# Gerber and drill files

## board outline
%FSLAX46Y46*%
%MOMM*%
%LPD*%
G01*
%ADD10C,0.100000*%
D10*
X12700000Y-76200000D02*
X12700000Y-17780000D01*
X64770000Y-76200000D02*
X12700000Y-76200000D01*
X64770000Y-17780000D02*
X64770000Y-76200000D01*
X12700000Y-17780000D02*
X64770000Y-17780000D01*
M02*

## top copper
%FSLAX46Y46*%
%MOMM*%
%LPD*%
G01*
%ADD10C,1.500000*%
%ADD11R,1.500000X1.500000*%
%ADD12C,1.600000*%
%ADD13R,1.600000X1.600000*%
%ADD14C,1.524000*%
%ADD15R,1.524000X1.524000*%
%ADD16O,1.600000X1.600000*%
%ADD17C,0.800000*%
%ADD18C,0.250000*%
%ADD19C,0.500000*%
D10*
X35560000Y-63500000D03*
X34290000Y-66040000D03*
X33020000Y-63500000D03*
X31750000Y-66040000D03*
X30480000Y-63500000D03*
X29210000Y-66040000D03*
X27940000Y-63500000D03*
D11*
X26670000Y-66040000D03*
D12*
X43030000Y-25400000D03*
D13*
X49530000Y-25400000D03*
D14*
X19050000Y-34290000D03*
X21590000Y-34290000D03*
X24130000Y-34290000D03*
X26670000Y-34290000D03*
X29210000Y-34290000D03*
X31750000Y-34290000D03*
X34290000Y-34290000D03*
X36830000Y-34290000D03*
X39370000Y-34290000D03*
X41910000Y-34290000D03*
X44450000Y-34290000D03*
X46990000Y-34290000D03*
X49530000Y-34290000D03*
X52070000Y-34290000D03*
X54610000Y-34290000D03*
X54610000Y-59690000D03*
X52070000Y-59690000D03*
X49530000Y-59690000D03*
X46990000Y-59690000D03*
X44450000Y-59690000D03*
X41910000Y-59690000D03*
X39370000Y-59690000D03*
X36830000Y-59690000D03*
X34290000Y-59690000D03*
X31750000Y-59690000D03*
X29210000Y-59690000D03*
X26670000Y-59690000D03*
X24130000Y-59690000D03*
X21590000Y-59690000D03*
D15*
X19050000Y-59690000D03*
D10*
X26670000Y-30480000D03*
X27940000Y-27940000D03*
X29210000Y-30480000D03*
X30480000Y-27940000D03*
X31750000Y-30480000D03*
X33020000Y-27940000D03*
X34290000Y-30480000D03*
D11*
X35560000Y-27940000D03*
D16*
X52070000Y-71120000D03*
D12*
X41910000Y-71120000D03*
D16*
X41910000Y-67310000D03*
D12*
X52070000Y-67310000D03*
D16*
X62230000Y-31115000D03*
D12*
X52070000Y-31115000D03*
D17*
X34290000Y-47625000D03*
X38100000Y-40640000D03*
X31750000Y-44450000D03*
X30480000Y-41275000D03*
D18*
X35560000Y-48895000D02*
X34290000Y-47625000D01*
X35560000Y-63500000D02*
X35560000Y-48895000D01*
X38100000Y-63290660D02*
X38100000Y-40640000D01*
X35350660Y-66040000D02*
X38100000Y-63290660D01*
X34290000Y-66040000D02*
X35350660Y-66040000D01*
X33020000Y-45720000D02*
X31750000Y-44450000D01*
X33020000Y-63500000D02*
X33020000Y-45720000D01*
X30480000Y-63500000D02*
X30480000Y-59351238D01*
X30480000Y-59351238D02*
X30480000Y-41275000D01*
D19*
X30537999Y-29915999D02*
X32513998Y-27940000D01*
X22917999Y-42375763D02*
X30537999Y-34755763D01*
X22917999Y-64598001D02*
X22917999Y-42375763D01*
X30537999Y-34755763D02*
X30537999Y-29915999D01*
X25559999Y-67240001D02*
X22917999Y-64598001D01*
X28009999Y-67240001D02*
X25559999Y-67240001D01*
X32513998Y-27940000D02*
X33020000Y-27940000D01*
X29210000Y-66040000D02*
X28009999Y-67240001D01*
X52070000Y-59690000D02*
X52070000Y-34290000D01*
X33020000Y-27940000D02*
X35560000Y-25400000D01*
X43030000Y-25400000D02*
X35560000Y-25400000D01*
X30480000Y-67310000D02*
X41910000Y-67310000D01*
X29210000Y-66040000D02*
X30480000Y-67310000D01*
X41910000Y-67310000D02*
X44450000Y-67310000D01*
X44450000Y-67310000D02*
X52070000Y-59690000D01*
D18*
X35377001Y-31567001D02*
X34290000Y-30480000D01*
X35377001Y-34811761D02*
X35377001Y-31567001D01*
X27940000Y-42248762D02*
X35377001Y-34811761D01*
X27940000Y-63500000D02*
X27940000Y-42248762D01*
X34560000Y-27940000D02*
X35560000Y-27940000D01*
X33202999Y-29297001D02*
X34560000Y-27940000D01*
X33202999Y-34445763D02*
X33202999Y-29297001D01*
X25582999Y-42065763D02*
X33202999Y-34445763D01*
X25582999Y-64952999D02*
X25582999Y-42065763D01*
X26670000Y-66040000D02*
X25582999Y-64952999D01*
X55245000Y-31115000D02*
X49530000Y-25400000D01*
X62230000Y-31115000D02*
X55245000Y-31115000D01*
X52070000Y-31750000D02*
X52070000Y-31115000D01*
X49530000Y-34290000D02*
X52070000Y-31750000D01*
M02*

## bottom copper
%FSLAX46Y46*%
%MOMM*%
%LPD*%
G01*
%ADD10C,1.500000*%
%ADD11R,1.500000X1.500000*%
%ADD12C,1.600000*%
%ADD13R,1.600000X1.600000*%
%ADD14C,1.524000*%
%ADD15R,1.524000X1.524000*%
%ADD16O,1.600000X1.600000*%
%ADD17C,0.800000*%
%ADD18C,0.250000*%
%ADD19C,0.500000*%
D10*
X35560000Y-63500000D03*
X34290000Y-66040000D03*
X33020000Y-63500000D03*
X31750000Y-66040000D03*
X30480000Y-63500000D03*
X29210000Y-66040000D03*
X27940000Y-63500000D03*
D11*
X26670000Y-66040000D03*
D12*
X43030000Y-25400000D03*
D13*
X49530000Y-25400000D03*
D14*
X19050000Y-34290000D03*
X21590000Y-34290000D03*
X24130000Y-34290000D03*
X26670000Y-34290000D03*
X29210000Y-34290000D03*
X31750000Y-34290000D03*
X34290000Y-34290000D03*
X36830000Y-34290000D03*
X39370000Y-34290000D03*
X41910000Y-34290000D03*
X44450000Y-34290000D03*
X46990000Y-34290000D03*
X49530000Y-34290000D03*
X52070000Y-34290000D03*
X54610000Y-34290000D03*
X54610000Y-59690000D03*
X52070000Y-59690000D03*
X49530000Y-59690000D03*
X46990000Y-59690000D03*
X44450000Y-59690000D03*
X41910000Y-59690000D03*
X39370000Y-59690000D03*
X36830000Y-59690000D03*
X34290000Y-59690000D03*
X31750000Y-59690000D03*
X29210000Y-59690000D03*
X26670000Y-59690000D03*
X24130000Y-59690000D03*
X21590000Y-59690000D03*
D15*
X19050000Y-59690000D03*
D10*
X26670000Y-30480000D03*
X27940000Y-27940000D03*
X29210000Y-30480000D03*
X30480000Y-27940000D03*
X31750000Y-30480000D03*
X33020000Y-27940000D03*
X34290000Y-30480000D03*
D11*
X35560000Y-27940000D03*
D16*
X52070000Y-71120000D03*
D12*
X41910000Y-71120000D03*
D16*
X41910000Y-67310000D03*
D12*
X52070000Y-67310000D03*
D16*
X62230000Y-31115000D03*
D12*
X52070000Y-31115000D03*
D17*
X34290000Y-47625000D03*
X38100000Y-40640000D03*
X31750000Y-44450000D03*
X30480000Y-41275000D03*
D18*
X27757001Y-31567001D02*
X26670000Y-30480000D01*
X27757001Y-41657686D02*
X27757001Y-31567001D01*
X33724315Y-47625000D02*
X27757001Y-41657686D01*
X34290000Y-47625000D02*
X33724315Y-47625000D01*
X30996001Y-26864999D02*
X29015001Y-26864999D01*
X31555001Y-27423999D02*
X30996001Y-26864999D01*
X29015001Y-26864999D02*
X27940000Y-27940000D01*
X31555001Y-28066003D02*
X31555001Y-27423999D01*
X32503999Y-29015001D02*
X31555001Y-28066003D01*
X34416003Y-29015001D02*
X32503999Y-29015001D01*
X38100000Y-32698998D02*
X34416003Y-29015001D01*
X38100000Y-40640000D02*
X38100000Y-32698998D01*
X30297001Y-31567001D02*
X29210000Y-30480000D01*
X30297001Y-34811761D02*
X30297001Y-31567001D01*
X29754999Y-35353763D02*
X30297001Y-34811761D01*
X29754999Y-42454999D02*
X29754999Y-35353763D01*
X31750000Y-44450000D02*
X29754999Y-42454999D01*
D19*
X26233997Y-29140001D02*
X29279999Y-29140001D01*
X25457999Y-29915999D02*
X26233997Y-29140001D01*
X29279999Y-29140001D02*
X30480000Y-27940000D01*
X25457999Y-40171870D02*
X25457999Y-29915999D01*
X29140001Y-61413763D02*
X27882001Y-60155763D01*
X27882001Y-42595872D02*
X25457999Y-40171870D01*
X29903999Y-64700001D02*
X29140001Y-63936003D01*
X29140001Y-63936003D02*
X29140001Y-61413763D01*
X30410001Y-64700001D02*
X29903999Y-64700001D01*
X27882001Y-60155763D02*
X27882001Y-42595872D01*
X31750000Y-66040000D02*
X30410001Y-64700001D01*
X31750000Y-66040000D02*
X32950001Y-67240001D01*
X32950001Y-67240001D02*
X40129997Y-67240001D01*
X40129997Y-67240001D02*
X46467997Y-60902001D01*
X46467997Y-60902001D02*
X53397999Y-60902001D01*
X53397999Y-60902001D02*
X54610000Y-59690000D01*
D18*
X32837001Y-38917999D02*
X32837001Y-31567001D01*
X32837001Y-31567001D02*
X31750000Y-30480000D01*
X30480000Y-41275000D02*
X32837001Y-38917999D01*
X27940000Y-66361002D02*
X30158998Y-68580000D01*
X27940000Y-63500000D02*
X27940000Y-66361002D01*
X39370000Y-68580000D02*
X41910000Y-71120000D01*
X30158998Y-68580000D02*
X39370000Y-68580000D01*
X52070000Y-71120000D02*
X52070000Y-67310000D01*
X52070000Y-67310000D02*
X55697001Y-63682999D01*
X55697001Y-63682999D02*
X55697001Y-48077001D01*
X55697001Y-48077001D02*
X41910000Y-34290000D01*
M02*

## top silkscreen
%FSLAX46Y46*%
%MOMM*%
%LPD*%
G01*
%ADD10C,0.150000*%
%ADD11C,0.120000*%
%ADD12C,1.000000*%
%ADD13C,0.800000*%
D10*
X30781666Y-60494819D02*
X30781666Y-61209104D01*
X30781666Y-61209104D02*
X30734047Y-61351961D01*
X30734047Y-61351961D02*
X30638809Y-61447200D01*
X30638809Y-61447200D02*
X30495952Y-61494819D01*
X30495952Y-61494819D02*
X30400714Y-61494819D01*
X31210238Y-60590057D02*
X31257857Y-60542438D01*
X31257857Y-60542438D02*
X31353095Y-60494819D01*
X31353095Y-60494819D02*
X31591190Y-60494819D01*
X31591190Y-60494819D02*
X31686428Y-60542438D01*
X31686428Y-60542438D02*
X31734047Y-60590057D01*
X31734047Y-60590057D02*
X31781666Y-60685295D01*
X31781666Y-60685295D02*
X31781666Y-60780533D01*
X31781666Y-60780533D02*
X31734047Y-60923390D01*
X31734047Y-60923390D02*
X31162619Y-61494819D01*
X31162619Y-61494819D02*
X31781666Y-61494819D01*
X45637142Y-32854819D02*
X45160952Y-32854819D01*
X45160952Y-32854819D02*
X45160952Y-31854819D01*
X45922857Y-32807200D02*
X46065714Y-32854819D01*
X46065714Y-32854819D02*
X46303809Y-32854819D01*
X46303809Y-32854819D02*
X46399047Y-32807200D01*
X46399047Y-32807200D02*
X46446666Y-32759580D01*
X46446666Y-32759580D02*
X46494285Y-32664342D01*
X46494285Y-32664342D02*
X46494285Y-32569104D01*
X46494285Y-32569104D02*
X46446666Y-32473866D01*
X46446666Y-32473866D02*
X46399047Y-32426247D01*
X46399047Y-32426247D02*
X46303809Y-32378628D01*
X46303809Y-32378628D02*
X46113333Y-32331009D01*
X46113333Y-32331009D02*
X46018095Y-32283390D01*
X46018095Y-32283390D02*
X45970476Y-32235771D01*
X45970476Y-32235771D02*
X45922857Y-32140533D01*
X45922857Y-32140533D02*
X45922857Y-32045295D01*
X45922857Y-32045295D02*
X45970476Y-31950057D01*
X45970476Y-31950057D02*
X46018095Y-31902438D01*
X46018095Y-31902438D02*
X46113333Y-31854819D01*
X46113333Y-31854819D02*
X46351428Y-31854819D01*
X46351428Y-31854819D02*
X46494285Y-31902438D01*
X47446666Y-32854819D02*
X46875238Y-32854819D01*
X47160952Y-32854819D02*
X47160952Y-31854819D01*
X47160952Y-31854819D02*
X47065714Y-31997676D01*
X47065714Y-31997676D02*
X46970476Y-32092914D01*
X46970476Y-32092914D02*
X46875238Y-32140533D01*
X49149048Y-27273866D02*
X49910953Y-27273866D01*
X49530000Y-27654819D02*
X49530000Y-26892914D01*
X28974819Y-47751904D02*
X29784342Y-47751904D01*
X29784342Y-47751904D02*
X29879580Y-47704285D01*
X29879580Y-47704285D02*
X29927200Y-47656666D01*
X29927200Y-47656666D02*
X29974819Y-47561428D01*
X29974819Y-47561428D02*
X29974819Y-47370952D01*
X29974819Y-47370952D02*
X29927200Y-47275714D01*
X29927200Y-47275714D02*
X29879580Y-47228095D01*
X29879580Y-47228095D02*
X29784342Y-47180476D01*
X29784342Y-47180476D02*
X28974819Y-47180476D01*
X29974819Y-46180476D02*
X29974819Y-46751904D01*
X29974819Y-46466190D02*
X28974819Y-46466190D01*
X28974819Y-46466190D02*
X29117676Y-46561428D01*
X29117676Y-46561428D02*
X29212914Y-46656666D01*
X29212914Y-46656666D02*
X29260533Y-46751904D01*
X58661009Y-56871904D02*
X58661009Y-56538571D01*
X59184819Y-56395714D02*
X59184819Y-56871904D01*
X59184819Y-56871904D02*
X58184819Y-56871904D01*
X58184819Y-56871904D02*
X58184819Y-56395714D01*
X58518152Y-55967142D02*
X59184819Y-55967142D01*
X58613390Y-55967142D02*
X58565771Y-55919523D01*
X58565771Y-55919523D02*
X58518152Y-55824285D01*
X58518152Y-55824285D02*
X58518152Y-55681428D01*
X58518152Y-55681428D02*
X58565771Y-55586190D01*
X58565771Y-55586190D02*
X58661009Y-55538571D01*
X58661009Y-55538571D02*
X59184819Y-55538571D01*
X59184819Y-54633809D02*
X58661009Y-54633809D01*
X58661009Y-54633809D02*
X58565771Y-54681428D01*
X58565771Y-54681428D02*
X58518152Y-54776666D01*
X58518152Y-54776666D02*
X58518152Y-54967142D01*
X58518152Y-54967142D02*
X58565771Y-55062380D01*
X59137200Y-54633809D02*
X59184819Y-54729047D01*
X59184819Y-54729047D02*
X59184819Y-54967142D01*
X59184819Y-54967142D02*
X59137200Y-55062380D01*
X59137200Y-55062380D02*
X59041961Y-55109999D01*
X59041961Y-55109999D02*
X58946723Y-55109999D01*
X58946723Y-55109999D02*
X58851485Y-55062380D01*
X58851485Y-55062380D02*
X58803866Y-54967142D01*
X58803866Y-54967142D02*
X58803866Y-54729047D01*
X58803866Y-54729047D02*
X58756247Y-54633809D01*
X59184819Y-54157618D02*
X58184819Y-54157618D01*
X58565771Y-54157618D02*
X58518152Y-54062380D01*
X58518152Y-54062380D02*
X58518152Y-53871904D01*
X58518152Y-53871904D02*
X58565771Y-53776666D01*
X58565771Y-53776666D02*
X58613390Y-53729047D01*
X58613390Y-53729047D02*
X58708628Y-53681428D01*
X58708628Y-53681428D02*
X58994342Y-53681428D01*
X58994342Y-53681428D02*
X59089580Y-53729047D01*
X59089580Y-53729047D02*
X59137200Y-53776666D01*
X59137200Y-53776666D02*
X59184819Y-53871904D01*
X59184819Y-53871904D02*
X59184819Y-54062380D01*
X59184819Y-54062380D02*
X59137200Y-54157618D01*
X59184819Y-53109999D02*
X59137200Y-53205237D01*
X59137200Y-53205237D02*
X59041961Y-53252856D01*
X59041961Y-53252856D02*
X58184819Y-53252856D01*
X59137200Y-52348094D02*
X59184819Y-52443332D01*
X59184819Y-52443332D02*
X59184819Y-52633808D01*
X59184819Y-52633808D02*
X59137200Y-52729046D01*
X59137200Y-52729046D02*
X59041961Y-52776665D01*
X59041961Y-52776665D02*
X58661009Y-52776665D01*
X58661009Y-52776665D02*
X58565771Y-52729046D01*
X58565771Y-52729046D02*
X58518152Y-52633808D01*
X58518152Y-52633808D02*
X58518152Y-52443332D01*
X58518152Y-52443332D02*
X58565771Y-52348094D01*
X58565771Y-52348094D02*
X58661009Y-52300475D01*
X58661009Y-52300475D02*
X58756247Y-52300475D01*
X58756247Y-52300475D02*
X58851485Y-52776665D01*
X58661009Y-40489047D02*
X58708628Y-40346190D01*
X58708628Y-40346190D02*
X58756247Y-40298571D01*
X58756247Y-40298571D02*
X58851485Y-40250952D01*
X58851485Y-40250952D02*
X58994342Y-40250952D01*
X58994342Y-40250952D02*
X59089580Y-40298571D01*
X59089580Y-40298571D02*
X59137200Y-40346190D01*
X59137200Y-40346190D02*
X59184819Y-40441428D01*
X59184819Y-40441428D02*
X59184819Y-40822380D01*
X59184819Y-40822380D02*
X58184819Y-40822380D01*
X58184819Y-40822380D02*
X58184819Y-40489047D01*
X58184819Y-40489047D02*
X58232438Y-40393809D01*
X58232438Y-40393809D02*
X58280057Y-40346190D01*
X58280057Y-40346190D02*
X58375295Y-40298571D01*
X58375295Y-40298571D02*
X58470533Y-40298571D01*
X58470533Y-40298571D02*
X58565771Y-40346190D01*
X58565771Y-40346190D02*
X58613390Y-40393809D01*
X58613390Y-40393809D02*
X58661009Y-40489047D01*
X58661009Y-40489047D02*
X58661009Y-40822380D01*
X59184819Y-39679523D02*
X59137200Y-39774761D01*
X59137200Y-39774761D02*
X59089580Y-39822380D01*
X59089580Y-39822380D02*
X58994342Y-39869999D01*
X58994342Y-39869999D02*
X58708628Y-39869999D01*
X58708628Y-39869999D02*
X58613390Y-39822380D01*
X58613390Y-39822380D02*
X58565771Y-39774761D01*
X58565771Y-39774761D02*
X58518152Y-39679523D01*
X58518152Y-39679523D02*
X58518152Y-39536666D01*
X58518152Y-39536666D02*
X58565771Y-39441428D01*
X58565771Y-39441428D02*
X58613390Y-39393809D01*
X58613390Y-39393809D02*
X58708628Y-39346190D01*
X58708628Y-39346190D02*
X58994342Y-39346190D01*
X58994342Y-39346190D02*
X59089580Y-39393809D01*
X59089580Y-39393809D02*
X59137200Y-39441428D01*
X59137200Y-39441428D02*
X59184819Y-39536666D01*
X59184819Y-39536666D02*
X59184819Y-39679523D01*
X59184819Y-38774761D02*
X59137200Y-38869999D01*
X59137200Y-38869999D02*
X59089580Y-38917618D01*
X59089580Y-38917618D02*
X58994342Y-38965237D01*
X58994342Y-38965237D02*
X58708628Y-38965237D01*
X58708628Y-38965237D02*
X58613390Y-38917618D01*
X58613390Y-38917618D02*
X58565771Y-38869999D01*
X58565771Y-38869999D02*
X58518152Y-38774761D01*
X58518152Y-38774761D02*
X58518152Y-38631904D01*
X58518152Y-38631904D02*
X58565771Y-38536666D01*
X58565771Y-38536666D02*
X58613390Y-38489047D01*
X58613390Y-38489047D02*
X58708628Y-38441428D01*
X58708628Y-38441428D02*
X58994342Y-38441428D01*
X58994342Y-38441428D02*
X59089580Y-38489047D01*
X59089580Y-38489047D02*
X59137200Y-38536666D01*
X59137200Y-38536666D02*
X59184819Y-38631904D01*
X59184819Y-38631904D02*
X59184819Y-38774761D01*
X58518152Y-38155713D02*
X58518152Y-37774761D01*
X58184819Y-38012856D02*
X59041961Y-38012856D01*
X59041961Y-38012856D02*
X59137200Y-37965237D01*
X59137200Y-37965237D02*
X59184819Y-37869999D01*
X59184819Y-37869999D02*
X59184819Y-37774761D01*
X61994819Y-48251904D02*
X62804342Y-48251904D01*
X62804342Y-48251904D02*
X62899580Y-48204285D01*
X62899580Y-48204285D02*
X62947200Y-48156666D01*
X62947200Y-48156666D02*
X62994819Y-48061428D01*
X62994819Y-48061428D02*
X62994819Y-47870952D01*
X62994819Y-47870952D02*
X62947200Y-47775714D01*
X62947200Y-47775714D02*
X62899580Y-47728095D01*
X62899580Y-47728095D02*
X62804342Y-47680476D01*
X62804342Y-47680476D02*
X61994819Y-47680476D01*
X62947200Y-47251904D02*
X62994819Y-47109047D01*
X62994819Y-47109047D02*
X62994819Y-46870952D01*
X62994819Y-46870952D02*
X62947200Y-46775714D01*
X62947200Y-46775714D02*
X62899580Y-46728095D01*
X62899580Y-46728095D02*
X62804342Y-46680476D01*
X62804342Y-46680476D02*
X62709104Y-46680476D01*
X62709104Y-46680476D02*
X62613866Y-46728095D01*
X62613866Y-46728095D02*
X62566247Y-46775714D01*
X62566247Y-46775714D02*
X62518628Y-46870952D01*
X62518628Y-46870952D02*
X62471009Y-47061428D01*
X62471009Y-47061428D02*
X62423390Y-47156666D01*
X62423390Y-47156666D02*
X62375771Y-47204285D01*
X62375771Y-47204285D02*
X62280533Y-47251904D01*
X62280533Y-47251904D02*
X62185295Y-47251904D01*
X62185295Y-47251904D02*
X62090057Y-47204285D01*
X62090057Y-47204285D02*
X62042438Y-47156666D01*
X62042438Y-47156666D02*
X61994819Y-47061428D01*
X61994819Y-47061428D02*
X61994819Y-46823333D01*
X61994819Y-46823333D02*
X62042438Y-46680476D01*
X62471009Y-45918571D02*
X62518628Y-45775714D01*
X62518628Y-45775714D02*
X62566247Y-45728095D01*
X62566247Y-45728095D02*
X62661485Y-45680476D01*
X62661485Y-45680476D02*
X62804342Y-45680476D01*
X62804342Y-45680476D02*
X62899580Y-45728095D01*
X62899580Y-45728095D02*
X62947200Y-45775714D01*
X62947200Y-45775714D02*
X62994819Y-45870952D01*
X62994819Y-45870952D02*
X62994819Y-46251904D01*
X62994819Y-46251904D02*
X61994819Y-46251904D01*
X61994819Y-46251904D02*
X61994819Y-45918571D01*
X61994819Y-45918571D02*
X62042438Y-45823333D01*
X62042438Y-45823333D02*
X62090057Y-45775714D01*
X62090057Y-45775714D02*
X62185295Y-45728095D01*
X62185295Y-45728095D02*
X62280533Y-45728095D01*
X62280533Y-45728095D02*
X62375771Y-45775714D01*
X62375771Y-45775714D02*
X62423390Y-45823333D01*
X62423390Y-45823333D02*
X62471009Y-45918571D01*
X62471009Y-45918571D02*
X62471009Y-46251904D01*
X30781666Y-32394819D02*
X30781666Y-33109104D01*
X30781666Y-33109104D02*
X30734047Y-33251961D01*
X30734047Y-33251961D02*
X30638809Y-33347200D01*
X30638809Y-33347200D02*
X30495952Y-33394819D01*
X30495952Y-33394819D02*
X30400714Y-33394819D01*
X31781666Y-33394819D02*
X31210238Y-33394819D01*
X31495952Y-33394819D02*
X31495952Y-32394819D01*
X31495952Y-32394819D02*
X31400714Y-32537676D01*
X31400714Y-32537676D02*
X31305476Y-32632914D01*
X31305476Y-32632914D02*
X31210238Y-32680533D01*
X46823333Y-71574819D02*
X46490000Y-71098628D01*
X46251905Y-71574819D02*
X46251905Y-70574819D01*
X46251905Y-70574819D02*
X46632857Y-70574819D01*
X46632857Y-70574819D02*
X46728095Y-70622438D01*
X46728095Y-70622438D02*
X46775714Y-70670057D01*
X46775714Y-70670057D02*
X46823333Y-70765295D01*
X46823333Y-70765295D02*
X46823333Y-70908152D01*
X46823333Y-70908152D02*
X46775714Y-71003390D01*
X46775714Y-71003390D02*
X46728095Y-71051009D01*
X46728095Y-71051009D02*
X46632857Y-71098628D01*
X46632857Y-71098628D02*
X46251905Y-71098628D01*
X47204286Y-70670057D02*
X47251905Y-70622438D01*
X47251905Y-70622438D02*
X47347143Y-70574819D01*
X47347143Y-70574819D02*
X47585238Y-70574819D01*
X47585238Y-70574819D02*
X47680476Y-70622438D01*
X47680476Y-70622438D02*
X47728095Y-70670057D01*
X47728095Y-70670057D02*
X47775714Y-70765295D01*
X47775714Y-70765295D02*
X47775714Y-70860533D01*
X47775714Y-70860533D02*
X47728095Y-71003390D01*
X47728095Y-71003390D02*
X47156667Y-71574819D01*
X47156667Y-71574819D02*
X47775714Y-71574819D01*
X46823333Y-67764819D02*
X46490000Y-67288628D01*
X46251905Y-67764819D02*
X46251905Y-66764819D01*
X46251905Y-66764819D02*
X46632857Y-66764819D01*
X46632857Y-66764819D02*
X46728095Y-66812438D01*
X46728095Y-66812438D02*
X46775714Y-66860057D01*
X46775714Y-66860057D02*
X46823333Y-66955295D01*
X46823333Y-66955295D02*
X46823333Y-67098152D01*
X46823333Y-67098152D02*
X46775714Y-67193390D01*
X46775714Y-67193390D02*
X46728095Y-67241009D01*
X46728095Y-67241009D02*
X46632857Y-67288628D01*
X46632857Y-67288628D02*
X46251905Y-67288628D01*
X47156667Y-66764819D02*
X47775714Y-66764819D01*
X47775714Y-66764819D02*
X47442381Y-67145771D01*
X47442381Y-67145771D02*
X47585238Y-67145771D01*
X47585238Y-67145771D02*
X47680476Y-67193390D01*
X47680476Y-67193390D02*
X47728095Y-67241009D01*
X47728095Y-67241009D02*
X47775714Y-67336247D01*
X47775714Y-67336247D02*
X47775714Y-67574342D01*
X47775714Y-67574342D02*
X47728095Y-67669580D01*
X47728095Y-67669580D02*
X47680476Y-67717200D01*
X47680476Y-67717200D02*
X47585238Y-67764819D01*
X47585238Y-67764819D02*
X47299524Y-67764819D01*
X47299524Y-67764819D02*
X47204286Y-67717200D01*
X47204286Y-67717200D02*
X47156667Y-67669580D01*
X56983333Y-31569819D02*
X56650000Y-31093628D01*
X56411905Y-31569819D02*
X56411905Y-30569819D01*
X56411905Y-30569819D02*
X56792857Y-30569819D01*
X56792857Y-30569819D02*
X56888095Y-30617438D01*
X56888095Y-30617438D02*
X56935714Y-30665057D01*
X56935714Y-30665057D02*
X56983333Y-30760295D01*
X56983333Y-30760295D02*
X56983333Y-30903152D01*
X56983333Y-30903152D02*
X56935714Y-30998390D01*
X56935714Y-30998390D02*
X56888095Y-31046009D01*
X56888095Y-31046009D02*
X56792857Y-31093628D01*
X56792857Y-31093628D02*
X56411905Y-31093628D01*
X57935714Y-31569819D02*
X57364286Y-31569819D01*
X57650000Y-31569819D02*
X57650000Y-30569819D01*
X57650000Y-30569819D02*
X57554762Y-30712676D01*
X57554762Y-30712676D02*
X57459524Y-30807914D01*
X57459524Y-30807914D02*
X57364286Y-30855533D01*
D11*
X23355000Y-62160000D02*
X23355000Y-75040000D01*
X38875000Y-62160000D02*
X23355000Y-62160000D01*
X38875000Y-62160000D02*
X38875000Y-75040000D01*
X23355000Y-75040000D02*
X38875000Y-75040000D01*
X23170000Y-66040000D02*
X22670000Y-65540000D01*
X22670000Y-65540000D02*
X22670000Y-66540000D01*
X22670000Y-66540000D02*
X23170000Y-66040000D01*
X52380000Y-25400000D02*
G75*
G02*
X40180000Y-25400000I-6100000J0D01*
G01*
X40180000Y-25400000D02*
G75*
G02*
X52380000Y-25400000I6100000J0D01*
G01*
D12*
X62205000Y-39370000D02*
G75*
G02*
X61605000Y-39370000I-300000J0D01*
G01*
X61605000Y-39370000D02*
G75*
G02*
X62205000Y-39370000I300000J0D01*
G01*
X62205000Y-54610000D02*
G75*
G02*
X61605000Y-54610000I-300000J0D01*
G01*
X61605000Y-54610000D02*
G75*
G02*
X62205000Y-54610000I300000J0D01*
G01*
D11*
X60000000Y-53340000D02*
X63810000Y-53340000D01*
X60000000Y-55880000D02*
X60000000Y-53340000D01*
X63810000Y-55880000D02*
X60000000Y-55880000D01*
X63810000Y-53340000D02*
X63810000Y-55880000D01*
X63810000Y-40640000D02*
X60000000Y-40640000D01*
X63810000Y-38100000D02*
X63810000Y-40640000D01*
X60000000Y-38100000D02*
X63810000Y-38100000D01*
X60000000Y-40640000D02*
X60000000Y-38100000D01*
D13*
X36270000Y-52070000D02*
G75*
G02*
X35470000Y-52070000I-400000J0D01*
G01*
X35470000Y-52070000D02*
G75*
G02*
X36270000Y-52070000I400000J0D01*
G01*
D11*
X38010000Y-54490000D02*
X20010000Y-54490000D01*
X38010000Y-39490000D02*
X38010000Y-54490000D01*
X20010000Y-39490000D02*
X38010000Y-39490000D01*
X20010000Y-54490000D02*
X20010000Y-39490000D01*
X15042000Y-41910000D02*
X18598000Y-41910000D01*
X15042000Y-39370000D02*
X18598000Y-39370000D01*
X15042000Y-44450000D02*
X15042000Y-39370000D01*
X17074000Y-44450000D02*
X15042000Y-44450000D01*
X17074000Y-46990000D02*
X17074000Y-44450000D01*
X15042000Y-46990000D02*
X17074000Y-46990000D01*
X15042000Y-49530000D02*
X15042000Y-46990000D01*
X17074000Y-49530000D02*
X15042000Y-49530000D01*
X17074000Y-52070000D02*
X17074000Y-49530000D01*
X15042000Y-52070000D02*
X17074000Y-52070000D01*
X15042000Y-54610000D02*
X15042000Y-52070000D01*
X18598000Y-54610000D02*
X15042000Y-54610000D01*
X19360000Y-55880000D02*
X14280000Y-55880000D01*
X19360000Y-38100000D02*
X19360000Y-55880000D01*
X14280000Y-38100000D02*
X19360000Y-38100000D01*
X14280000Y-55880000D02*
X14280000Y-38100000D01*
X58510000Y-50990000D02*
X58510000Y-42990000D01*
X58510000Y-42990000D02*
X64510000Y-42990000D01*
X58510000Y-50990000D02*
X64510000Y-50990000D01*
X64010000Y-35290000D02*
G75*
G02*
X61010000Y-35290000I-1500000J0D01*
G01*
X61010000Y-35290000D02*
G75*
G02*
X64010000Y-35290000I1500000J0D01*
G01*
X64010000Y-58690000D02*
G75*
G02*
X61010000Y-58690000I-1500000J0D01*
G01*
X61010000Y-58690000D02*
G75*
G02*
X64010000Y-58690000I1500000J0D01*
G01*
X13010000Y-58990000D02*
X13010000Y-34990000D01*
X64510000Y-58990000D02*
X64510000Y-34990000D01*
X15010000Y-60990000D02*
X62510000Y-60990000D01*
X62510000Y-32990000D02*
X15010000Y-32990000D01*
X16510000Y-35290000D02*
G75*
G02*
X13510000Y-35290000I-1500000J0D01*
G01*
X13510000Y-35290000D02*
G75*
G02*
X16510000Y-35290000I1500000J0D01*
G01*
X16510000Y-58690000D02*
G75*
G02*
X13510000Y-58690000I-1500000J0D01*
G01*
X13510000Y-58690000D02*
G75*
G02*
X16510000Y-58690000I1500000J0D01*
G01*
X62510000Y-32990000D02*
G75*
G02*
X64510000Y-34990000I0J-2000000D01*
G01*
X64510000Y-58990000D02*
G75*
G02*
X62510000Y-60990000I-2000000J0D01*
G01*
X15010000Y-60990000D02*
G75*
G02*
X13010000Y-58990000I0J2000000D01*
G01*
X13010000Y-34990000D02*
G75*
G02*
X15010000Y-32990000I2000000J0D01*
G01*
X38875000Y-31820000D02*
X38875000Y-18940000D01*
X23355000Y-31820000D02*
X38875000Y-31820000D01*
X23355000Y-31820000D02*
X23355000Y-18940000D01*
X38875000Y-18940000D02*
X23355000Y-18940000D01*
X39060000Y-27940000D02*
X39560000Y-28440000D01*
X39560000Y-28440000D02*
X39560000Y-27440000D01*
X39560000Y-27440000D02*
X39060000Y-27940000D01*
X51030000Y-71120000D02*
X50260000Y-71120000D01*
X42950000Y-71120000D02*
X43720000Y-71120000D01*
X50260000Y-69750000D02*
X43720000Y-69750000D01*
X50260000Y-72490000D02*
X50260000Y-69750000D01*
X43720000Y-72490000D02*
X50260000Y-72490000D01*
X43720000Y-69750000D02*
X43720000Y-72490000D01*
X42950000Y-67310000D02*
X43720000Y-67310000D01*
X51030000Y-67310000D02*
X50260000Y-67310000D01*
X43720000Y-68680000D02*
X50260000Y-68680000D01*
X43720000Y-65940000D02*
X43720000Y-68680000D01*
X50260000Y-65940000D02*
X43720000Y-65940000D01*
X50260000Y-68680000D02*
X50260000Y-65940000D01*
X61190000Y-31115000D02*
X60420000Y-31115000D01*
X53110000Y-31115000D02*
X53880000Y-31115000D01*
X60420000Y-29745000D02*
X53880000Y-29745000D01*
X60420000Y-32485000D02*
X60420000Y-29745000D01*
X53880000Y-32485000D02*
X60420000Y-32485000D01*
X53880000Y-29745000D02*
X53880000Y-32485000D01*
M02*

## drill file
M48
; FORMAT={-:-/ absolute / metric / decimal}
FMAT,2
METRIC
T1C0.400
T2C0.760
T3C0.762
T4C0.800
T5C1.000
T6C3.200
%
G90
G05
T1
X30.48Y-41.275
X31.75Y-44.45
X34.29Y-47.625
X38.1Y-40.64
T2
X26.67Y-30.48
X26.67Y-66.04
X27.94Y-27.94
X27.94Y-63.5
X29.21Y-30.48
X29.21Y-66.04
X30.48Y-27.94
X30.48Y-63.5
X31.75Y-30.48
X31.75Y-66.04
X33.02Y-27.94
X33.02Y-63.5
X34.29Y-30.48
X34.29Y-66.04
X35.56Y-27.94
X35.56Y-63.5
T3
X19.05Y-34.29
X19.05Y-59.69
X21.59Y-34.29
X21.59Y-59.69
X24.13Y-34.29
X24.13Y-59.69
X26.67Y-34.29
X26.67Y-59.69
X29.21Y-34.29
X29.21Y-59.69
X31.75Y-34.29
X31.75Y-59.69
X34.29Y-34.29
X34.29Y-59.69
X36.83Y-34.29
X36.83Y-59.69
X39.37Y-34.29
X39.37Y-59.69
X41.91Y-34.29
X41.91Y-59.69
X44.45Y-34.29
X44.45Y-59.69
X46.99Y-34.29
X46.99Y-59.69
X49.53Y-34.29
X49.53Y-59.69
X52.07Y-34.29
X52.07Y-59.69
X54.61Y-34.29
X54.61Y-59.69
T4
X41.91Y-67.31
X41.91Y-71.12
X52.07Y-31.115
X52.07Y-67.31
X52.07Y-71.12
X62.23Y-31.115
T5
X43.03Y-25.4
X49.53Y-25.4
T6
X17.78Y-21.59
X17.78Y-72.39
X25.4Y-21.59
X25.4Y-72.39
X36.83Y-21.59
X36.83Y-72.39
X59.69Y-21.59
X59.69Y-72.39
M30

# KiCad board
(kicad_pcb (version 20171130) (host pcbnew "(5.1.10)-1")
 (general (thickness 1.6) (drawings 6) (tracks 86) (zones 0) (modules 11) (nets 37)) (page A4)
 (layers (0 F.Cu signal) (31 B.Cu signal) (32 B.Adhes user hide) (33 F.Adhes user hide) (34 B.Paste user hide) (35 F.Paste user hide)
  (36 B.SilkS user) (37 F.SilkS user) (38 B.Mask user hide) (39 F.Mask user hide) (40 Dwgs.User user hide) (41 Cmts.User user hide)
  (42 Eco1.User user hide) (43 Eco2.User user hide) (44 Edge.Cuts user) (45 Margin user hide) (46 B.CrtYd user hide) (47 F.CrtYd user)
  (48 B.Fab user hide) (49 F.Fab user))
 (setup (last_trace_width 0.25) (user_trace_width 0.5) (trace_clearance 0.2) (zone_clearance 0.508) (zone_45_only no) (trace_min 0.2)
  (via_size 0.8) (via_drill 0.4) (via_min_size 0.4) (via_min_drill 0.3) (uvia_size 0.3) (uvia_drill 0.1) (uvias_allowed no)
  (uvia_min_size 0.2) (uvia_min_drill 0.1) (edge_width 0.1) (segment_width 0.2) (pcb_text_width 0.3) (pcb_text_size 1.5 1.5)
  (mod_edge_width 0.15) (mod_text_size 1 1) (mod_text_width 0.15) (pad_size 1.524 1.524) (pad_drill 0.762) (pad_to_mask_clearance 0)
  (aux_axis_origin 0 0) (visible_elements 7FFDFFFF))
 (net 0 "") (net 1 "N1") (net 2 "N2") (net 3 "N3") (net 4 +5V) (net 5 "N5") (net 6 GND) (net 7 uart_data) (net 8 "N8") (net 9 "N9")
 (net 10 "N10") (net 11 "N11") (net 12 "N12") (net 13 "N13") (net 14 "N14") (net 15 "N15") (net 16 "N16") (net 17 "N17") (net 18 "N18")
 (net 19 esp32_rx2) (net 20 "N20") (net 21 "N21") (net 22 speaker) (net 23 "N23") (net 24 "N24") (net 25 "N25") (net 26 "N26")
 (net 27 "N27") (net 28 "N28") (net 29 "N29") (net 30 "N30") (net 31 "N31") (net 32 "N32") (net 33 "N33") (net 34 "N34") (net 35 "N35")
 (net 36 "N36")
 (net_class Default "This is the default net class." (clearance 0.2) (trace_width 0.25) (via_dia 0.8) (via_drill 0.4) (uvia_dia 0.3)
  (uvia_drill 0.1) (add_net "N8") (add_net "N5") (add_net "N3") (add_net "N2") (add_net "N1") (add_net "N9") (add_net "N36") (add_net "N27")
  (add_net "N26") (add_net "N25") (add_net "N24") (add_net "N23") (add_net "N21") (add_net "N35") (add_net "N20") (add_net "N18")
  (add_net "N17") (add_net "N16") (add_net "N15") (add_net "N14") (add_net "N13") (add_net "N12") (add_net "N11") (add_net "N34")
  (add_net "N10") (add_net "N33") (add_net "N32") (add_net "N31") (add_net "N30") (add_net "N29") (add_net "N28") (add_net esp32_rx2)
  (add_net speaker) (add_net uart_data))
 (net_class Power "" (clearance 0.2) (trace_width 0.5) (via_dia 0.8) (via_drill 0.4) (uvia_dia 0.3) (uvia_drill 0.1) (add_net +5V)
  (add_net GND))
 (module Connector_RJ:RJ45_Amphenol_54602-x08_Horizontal (layer F.Cu) (at 26.67 66.04)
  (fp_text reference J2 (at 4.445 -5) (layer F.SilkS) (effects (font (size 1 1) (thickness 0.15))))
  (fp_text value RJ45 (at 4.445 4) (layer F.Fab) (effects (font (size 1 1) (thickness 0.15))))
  (fp_line (start -3.315 -3.88) (end -3.315 9) (layer F.SilkS) (width 0.12))
  (fp_line (start 12.205 -3.88) (end -3.315 -3.88) (layer F.SilkS) (width 0.12))
  (fp_line (start 12.205 -3.88) (end 12.205 9) (layer F.SilkS) (width 0.12))
  (fp_line (start -3.315 9) (end 12.205 9) (layer F.SilkS) (width 0.12))
  (fp_line (start -3.5 0) (end -4 -0.5) (layer F.SilkS) (width 0.12))
  (fp_line (start -4 -0.5) (end -4 0.5) (layer F.SilkS) (width 0.12))
  (fp_line (start -4 0.5) (end -3.5 0) (layer F.SilkS) (width 0.12))
  (pad 8 thru_hole circle (at 8.89 -2.54) (size 1.5 1.5) (drill 0.76) (layers *.Cu *.Mask) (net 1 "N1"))
  (pad 7 thru_hole circle (at 7.62 0) (size 1.5 1.5) (drill 0.76) (layers *.Cu *.Mask) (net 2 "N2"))
  (pad 6 thru_hole circle (at 6.35 -2.54) (size 1.5 1.5) (drill 0.76) (layers *.Cu *.Mask) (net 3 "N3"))
  (pad 5 thru_hole circle (at 5.08 0) (size 1.5 1.5) (drill 0.76) (layers *.Cu *.Mask) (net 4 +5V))
  (pad 4 thru_hole circle (at 3.81 -2.54) (size 1.5 1.5) (drill 0.76) (layers *.Cu *.Mask) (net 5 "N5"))
  (pad 3 thru_hole circle (at 2.54 0) (size 1.5 1.5) (drill 0.76) (layers *.Cu *.Mask) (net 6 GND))
  (pad 2 thru_hole circle (at 1.27 -2.54) (size 1.5 1.5) (drill 0.76) (layers *.Cu *.Mask) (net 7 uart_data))
  (pad 1 thru_hole rect (at 0 0) (size 1.5 1.5) (drill 0.76) (layers *.Cu *.Mask) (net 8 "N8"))
  (pad "" np_thru_hole circle (at -1.27 6.35) (size 3.2 3.2) (drill 3.2) (layers *.Cu *.Mask))
  (pad "" np_thru_hole circle (at 10.16 6.35) (size 3.2 3.2) (drill 3.2) (layers *.Cu *.Mask)))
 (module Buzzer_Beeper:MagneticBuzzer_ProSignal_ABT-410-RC (layer F.Cu) (at 49.53 25.4 180)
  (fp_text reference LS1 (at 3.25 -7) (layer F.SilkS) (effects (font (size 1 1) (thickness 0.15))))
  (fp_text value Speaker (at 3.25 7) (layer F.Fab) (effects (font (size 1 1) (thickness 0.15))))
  (fp_circle (center 3.25 0) (end 9.35 0) (layer F.SilkS) (width 0.12))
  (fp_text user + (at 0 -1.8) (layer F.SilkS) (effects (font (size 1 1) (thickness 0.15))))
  (pad 2 thru_hole circle (at 6.5 0 180) (size 1.6 1.6) (drill 1) (layers *.Cu *.Mask) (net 6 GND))
  (pad 1 thru_hole rect (at 0 0 180) (size 1.6 1.6) (drill 1) (layers *.Cu *.Mask) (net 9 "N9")))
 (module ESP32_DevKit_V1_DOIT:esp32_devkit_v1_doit (layer F.Cu) (at 19.05 46.99 90)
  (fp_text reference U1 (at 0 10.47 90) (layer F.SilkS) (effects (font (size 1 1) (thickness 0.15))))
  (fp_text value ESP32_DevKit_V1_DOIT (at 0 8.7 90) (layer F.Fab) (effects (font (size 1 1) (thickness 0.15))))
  (fp_circle (center 7.62 42.855) (end 7.92 42.855) (layer F.SilkS) (width 1))
  (fp_circle (center -7.62 42.855) (end -7.32 42.855) (layer F.SilkS) (width 1))
  (fp_line (start -6.35 40.95) (end -6.35 44.76) (layer F.SilkS) (width 0.12))
  (fp_line (start -8.89 40.95) (end -6.35 40.95) (layer F.SilkS) (width 0.12))
  (fp_line (start -8.89 44.76) (end -8.89 40.95) (layer F.SilkS) (width 0.12))
  (fp_line (start -6.35 44.76) (end -8.89 44.76) (layer F.SilkS) (width 0.12))
  (fp_line (start 6.35 44.76) (end 6.35 40.95) (layer F.SilkS) (width 0.12))
  (fp_line (start 8.89 44.76) (end 6.35 44.76) (layer F.SilkS) (width 0.12))
  (fp_line (start 8.89 40.95) (end 8.89 44.76) (layer F.SilkS) (width 0.12))
  (fp_line (start 6.35 40.95) (end 8.89 40.95) (layer F.SilkS) (width 0.12))
  (fp_circle (center -5.08 16.82) (end -4.68 16.82) (layer F.SilkS) (width 0.8))
  (fp_line (start -7.5 18.96) (end -7.5 0.96) (layer F.SilkS) (width 0.12))
  (fp_line (start 7.5 18.96) (end -7.5 18.96) (layer F.SilkS) (width 0.12))
  (fp_line (start 7.5 0.96) (end 7.5 18.96) (layer F.SilkS) (width 0.12))
  (fp_line (start -7.5 0.96) (end 7.5 0.96) (layer F.SilkS) (width 0.12))
  (fp_line (start 5.08 -4.008) (end 5.08 -0.452) (layer F.SilkS) (width 0.12))
  (fp_line (start 7.62 -4.008) (end 7.62 -0.452) (layer F.SilkS) (width 0.12))
  (fp_line (start 2.54 -4.008) (end 7.62 -4.008) (layer F.SilkS) (width 0.12))
  (fp_line (start 2.54 -1.976) (end 2.54 -4.008) (layer F.SilkS) (width 0.12))
  (fp_line (start 0 -1.976) (end 2.54 -1.976) (layer F.SilkS) (width 0.12))
  (fp_line (start 0 -4.008) (end 0 -1.976) (layer F.SilkS) (width 0.12))
  (fp_line (start -2.54 -4.008) (end 0 -4.008) (layer F.SilkS) (width 0.12))
  (fp_line (start -2.54 -1.976) (end -2.54 -4.008) (layer F.SilkS) (width 0.12))
  (fp_line (start -5.08 -1.976) (end -2.54 -1.976) (layer F.SilkS) (width 0.12))
  (fp_line (start -5.08 -4.008) (end -5.08 -1.976) (layer F.SilkS) (width 0.12))
  (fp_line (start -7.62 -4.008) (end -5.08 -4.008) (layer F.SilkS) (width 0.12))
  (fp_line (start -7.62 -0.452) (end -7.62 -4.008) (layer F.SilkS) (width 0.12))
  (fp_line (start -8.89 0.31) (end -8.89 -4.77) (layer F.SilkS) (width 0.12))
  (fp_line (start 8.89 0.31) (end -8.89 0.31) (layer F.SilkS) (width 0.12))
  (fp_line (start 8.89 -4.77) (end 8.89 0.31) (layer F.SilkS) (width 0.12))
  (fp_line (start -8.89 -4.77) (end 8.89 -4.77) (layer F.SilkS) (width 0.12))
  (fp_line (start -4 39.46) (end 4 39.46) (layer F.SilkS) (width 0.12))
  (fp_line (start 4 39.46) (end 4 45.46) (layer F.SilkS) (width 0.12))
  (fp_line (start -4 39.46) (end -4 45.46) (layer F.SilkS) (width 0.12))
  (fp_circle (center 11.7 43.46) (end 13.2 43.46) (layer F.SilkS) (width 0.12))
  (fp_circle (center -11.7 43.46) (end -10.2 43.46) (layer F.SilkS) (width 0.12))
  (fp_line (start -12 -6.04) (end 12 -6.04) (layer F.SilkS) (width 0.12))
  (fp_line (start -12 45.46) (end 12 45.46) (layer F.SilkS) (width 0.12))
  (fp_line (start -14 -4.04) (end -14 43.46) (layer F.SilkS) (width 0.12))
  (fp_line (start 14 43.46) (end 14 -4.04) (layer F.SilkS) (width 0.12))
  (fp_circle (center 11.7 -4.04) (end 13.2 -4.04) (layer F.SilkS) (width 0.12))
  (fp_circle (center -11.7 -4.04) (end -10.2 -4.04) (layer F.SilkS) (width 0.12))
  (fp_arc (start 12 43.46) (end 12 45.46) (angle -90) (layer F.SilkS) (width 0.12))
  (fp_arc (start -12 43.46) (end -14 43.46) (angle -90) (layer F.SilkS) (width 0.12))
  (fp_arc (start -12 -4.04) (end -12 -6.04) (angle -90) (layer F.SilkS) (width 0.12))
  (fp_arc (start 12 -4.04) (end 14 -4.04) (angle -90) (layer F.SilkS) (width 0.12))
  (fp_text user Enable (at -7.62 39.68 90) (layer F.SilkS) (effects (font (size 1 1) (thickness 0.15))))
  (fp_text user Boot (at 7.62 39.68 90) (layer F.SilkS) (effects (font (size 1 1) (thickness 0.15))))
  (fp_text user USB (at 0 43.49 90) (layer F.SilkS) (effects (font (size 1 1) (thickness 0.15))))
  (pad 30 thru_hole circle (at 12.7 0 90) (size 1.524 1.524) (drill 0.762) (layers *.Cu *.Mask) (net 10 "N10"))
  (pad 29 thru_hole circle (at 12.7 2.54 90) (size 1.524 1.524) (drill 0.762) (layers *.Cu *.Mask) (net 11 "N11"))
  (pad 28 thru_hole circle (at 12.7 5.08 90) (size 1.524 1.524) (drill 0.762) (layers *.Cu *.Mask) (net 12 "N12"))
  (pad 27 thru_hole circle (at 12.7 7.62 90) (size 1.524 1.524) (drill 0.762) (layers *.Cu *.Mask) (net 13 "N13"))
  (pad 26 thru_hole circle (at 12.7 10.16 90) (size 1.524 1.524) (drill 0.762) (layers *.Cu *.Mask) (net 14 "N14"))
  (pad 25 thru_hole circle (at 12.7 12.7 90) (size 1.524 1.524) (drill 0.762) (layers *.Cu *.Mask) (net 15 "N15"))
  (pad 24 thru_hole circle (at 12.7 15.24 90) (size 1.524 1.524) (drill 0.762) (layers *.Cu *.Mask) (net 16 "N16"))
  (pad 23 thru_hole circle (at 12.7 17.78 90) (size 1.524 1.524) (drill 0.762) (layers *.Cu *.Mask) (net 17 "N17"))
  (pad 22 thru_hole circle (at 12.7 20.32 90) (size 1.524 1.524) (drill 0.762) (layers *.Cu *.Mask) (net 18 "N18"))
  (pad 21 thru_hole circle (at 12.7 22.86 90) (size 1.524 1.524) (drill 0.762) (layers *.Cu *.Mask) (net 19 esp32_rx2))
  (pad 20 thru_hole circle (at 12.7 25.4 90) (size 1.524 1.524) (drill 0.762) (layers *.Cu *.Mask) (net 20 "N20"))
  (pad 19 thru_hole circle (at 12.7 27.94 90) (size 1.524 1.524) (drill 0.762) (layers *.Cu *.Mask) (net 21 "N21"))
  (pad 18 thru_hole circle (at 12.7 30.48 90) (size 1.524 1.524) (drill 0.762) (layers *.Cu *.Mask) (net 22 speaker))
  (pad 17 thru_hole circle (at 12.7 33.02 90) (size 1.524 1.524) (drill 0.762) (layers *.Cu *.Mask) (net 6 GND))
  (pad 16 thru_hole circle (at 12.7 35.56 90) (size 1.524 1.524) (drill 0.762) (layers *.Cu *.Mask) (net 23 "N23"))
  (pad 15 thru_hole circle (at -12.7 35.56 90) (size 1.524 1.524) (drill 0.762) (layers *.Cu *.Mask) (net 4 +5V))
  (pad 14 thru_hole circle (at -12.7 33.02 90) (size 1.524 1.524) (drill 0.762) (layers *.Cu *.Mask) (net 6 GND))
  (pad 13 thru_hole circle (at -12.7 30.48 90) (size 1.524 1.524) (drill 0.762) (layers *.Cu *.Mask) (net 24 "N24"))
  (pad 12 thru_hole circle (at -12.7 27.94 90) (size 1.524 1.524) (drill 0.762) (layers *.Cu *.Mask) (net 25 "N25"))
  (pad 11 thru_hole circle (at -12.7 25.4 90) (size 1.524 1.524) (drill 0.762) (layers *.Cu *.Mask) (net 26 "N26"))
  (pad 10 thru_hole circle (at -12.7 22.86 90) (size 1.524 1.524) (drill 0.762) (layers *.Cu *.Mask) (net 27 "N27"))
  (pad 9 thru_hole circle (at -12.7 20.32 90) (size 1.524 1.524) (drill 0.762) (layers *.Cu *.Mask) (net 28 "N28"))
  (pad 8 thru_hole circle (at -12.7 17.78 90) (size 1.524 1.524) (drill 0.762) (layers *.Cu *.Mask) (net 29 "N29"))
  (pad 7 thru_hole circle (at -12.7 15.24 90) (size 1.524 1.524) (drill 0.762) (layers *.Cu *.Mask) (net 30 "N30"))
  (pad 6 thru_hole circle (at -12.7 12.7 90) (size 1.524 1.524) (drill 0.762) (layers *.Cu *.Mask) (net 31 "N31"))
  (pad 5 thru_hole circle (at -12.7 10.16 90) (size 1.524 1.524) (drill 0.762) (layers *.Cu *.Mask) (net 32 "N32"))
  (pad 4 thru_hole circle (at -12.7 7.62 90) (size 1.524 1.524) (drill 0.762) (layers *.Cu *.Mask) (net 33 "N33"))
  (pad 3 thru_hole circle (at -12.7 5.08 90) (size 1.524 1.524) (drill 0.762) (layers *.Cu *.Mask) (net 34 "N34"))
  (pad 2 thru_hole circle (at -12.7 2.54 90) (size 1.524 1.524) (drill 0.762) (layers *.Cu *.Mask) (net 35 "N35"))
  (pad 1 thru_hole rect (at -12.7 0 90) (size 1.524 1.524) (drill 0.762) (layers *.Cu *.Mask) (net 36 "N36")))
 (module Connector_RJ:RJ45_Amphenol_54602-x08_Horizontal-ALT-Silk (layer F.Cu) (at 35.56 27.94 180)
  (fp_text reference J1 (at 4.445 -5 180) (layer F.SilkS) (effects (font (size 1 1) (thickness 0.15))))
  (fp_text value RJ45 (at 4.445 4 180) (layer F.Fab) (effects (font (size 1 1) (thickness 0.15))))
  (fp_line (start -3.315 -3.88) (end -3.315 9) (layer F.SilkS) (width 0.12))
  (fp_line (start 12.205 -3.88) (end -3.315 -3.88) (layer F.SilkS) (width 0.12))
  (fp_line (start 12.205 -3.88) (end 12.205 9) (layer F.SilkS) (width 0.12))
  (fp_line (start -3.315 9) (end 12.205 9) (layer F.SilkS) (width 0.12))
  (fp_line (start -3.5 0) (end -4 -0.5) (layer F.SilkS) (width 0.12))
  (fp_line (start -4 -0.5) (end -4 0.5) (layer F.SilkS) (width 0.12))
  (fp_line (start -4 0.5) (end -3.5 0) (layer F.SilkS) (width 0.12))
  (pad 8 thru_hole circle (at 8.89 -2.54 180) (size 1.5 1.5) (drill 0.76) (layers *.Cu *.Mask) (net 1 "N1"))
  (pad 7 thru_hole circle (at 7.62 0 180) (size 1.5 1.5) (drill 0.76) (layers *.Cu *.Mask) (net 2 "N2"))
  (pad 6 thru_hole circle (at 6.35 -2.54 180) (size 1.5 1.5) (drill 0.76) (layers *.Cu *.Mask) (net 3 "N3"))
  (pad 5 thru_hole circle (at 5.08 0 180) (size 1.5 1.5) (drill 0.76) (layers *.Cu *.Mask) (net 4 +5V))
  (pad 4 thru_hole circle (at 3.81 -2.54 180) (size 1.5 1.5) (drill 0.76) (layers *.Cu *.Mask) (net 5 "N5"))
  (pad 3 thru_hole circle (at 2.54 0 180) (size 1.5 1.5) (drill 0.76) (layers *.Cu *.Mask) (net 6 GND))
  (pad 2 thru_hole circle (at 1.27 -2.54 180) (size 1.5 1.5) (drill 0.76) (layers *.Cu *.Mask) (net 7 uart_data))
  (pad 1 thru_hole rect (at 0 0 180) (size 1.5 1.5) (drill 0.76) (layers *.Cu *.Mask) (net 8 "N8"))
  (pad "" np_thru_hole circle (at -1.27 6.35 180) (size 3.2 3.2) (drill 3.2) (layers *.Cu *.Mask))
  (pad "" np_thru_hole circle (at 10.16 6.35 180) (size 3.2 3.2) (drill 3.2) (layers *.Cu *.Mask)))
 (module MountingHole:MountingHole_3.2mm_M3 (layer F.Cu) (at 17.78 72.39)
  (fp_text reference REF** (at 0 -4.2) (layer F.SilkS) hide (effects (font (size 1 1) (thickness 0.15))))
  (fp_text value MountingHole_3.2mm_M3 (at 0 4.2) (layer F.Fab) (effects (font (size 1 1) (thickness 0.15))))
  (pad 1 np_thru_hole circle (at 0 0) (size 3.2 3.2) (drill 3.2) (layers *.Cu *.Mask)))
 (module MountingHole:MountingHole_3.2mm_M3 (layer F.Cu) (at 59.69 21.59)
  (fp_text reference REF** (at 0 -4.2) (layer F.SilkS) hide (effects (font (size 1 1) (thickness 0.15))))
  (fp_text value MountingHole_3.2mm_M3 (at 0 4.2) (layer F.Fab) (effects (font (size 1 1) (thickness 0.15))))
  (pad 1 np_thru_hole circle (at 0 0) (size 3.2 3.2) (drill 3.2) (layers *.Cu *.Mask)))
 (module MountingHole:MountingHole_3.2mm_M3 (layer F.Cu) (at 17.78 21.59)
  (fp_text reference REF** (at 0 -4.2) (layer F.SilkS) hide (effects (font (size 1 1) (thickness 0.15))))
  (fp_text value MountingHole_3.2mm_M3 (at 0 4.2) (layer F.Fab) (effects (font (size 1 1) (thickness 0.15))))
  (pad 1 np_thru_hole circle (at 0 0) (size 3.2 3.2) (drill 3.2) (layers *.Cu *.Mask)))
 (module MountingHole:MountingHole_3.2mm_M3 (layer F.Cu) (at 59.69 72.39)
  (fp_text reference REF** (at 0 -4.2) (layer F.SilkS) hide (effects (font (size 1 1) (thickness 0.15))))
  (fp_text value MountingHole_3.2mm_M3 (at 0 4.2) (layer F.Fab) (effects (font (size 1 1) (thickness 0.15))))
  (pad 1 np_thru_hole circle (at 0 0) (size 3.2 3.2) (drill 3.2) (layers *.Cu *.Mask)))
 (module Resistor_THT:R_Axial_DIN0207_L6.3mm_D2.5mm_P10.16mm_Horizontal (layer F.Cu) (at 41.91 71.12)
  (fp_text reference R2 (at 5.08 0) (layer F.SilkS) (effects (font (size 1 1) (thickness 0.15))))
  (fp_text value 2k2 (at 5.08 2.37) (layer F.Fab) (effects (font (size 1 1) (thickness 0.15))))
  (fp_line (start 9.12 0) (end 8.35 0) (layer F.SilkS) (width 0.12))
  (fp_line (start 1.04 0) (end 1.81 0) (layer F.SilkS) (width 0.12))
  (fp_line (start 8.35 -1.37) (end 1.81 -1.37) (layer F.SilkS) (width 0.12))
  (fp_line (start 8.35 1.37) (end 8.35 -1.37) (layer F.SilkS) (width 0.12))
  (fp_line (start 1.81 1.37) (end 8.35 1.37) (layer F.SilkS) (width 0.12))
  (fp_line (start 1.81 -1.37) (end 1.81 1.37) (layer F.SilkS) (width 0.12))
  (pad 2 thru_hole oval (at 10.16 0) (size 1.6 1.6) (drill 0.8) (layers *.Cu *.Mask) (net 19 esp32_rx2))
  (pad 1 thru_hole circle (at 0 0) (size 1.6 1.6) (drill 0.8) (layers *.Cu *.Mask) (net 7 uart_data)))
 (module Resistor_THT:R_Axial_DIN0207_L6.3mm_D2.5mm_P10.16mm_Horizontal (layer F.Cu) (at 52.07 67.31 180)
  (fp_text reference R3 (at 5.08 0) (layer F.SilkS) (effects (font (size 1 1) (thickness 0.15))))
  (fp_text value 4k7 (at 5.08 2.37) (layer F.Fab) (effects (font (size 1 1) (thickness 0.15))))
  (fp_line (start 9.12 0) (end 8.35 0) (layer F.SilkS) (width 0.12))
  (fp_line (start 1.04 0) (end 1.81 0) (layer F.SilkS) (width 0.12))
  (fp_line (start 8.35 -1.37) (end 1.81 -1.37) (layer F.SilkS) (width 0.12))
  (fp_line (start 8.35 1.37) (end 8.35 -1.37) (layer F.SilkS) (width 0.12))
  (fp_line (start 1.81 1.37) (end 8.35 1.37) (layer F.SilkS) (width 0.12))
  (fp_line (start 1.81 -1.37) (end 1.81 1.37) (layer F.SilkS) (width 0.12))
  (pad 2 thru_hole oval (at 10.16 0 180) (size 1.6 1.6) (drill 0.8) (layers *.Cu *.Mask) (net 6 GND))
  (pad 1 thru_hole circle (at 0 0 180) (size 1.6 1.6) (drill 0.8) (layers *.Cu *.Mask) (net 19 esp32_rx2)))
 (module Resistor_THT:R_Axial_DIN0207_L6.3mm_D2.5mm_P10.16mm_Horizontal (layer F.Cu) (at 52.07 31.115)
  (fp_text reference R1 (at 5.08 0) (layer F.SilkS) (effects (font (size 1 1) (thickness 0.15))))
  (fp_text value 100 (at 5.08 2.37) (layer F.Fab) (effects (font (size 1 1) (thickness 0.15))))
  (fp_line (start 9.12 0) (end 8.35 0) (layer F.SilkS) (width 0.12))
  (fp_line (start 1.04 0) (end 1.81 0) (layer F.SilkS) (width 0.12))
  (fp_line (start 8.35 -1.37) (end 1.81 -1.37) (layer F.SilkS) (width 0.12))
  (fp_line (start 8.35 1.37) (end 8.35 -1.37) (layer F.SilkS) (width 0.12))
  (fp_line (start 1.81 1.37) (end 8.35 1.37) (layer F.SilkS) (width 0.12))
  (fp_line (start 1.81 -1.37) (end 1.81 1.37) (layer F.SilkS) (width 0.12))
  (pad 2 thru_hole oval (at 10.16 0) (size 1.6 1.6) (drill 0.8) (layers *.Cu *.Mask) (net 9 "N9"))
  (pad 1 thru_hole circle (at 0 0) (size 1.6 1.6) (drill 0.8) (layers *.Cu *.Mask) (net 22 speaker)))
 (gr_line (start 12.7 76.2) (end 12.7 17.78) (layer Edge.Cuts) (width 0.1))
 (gr_line (start 64.77 76.2) (end 12.7 76.2) (layer Edge.Cuts) (width 0.1))
 (gr_line (start 64.77 17.78) (end 64.77 76.2) (layer Edge.Cuts) (width 0.1))
 (gr_line (start 12.7 17.78) (end 64.77 17.78) (layer Edge.Cuts) (width 0.1))
 (via (at 34.29 47.625) (size 0.8) (drill 0.4) (layers F.Cu B.Cu) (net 1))
 (segment (start 35.56 48.895) (end 34.29 47.625) (width 0.25) (layer F.Cu) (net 1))
 (segment (start 35.56 63.5) (end 35.56 48.895) (width 0.25) (layer F.Cu) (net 1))
 (segment (start 27.757001 31.567001) (end 26.67 30.48) (width 0.25) (layer B.Cu) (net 1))
 (segment (start 27.757001 41.657686) (end 27.757001 31.567001) (width 0.25) (layer B.Cu) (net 1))
 (segment (start 33.724315 47.625) (end 27.757001 41.657686) (width 0.25) (layer B.Cu) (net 1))
 (segment (start 34.29 47.625) (end 33.724315 47.625) (width 0.25) (layer B.Cu) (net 1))
 (via (at 38.1 40.64) (size 0.8) (drill 0.4) (layers F.Cu B.Cu) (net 2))
 (segment (start 38.1 63.29066) (end 38.1 40.64) (width 0.25) (layer F.Cu) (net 2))
 (segment (start 35.35066 66.04) (end 38.1 63.29066) (width 0.25) (layer F.Cu) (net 2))
 (segment (start 34.29 66.04) (end 35.35066 66.04) (width 0.25) (layer F.Cu) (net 2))
 (segment (start 30.996001 26.864999) (end 29.015001 26.864999) (width 0.25) (layer B.Cu) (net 2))
 (segment (start 31.555001 27.423999) (end 30.996001 26.864999) (width 0.25) (layer B.Cu) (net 2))
 (segment (start 29.015001 26.864999) (end 27.94 27.94) (width 0.25) (layer B.Cu) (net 2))
 (segment (start 31.555001 28.066003) (end 31.555001 27.423999) (width 0.25) (layer B.Cu) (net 2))
 (segment (start 32.503999 29.015001) (end 31.555001 28.066003) (width 0.25) (layer B.Cu) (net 2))
 (segment (start 34.416003 29.015001) (end 32.503999 29.015001) (width 0.25) (layer B.Cu) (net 2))
 (segment (start 38.1 32.698998) (end 34.416003 29.015001) (width 0.25) (layer B.Cu) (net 2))
 (segment (start 38.1 40.64) (end 38.1 32.698998) (width 0.25) (layer B.Cu) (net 2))
 (via (at 31.75 44.45) (size 0.8) (drill 0.4) (layers F.Cu B.Cu) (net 3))
 (segment (start 33.02 45.72) (end 31.75 44.45) (width 0.25) (layer F.Cu) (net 3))
 (segment (start 33.02 63.5) (end 33.02 45.72) (width 0.25) (layer F.Cu) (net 3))
 (segment (start 30.297001 31.567001) (end 29.21 30.48) (width 0.25) (layer B.Cu) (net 3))
 (segment (start 30.297001 34.811761) (end 30.297001 31.567001) (width 0.25) (layer B.Cu) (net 3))
 (segment (start 29.754999 35.353763) (end 30.297001 34.811761) (width 0.25) (layer B.Cu) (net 3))
 (segment (start 29.754999 42.454999) (end 29.754999 35.353763) (width 0.25) (layer B.Cu) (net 3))
 (segment (start 31.75 44.45) (end 29.754999 42.454999) (width 0.25) (layer B.Cu) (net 3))
 (segment (start 26.233997 29.140001) (end 29.279999 29.140001) (width 0.5) (layer B.Cu) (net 4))
 (segment (start 25.457999 29.915999) (end 26.233997 29.140001) (width 0.5) (layer B.Cu) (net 4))
 (segment (start 29.279999 29.140001) (end 30.48 27.94) (width 0.5) (layer B.Cu) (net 4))
 (segment (start 25.457999 40.17187) (end 25.457999 29.915999) (width 0.5) (layer B.Cu) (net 4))
 (segment (start 29.140001 61.413763) (end 27.882001 60.155763) (width 0.5) (layer B.Cu) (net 4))
 (segment (start 27.882001 42.595872) (end 25.457999 40.17187) (width 0.5) (layer B.Cu) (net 4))
 (segment (start 29.903999 64.700001) (end 29.140001 63.936003) (width 0.5) (layer B.Cu) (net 4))
 (segment (start 29.140001 63.936003) (end 29.140001 61.413763) (width 0.5) (layer B.Cu) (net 4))
 (segment (start 30.410001 64.700001) (end 29.903999 64.700001) (width 0.5) (layer B.Cu) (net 4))
 (segment (start 27.882001 60.155763) (end 27.882001 42.595872) (width 0.5) (layer B.Cu) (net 4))
 (segment (start 31.75 66.04) (end 30.410001 64.700001) (width 0.5) (layer B.Cu) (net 4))
 (segment (start 31.75 66.04) (end 32.950001 67.240001) (width 0.5) (layer B.Cu) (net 4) (status 1000000))
 (segment (start 32.950001 67.240001) (end 40.129997 67.240001) (width 0.5) (layer B.Cu) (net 4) (status 1000000))
 (segment (start 40.129997 67.240001) (end 46.467997 60.902001) (width 0.5) (layer B.Cu) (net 4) (status 1000000))
 (segment (start 46.467997 60.902001) (end 53.397999 60.902001) (width 0.5) (layer B.Cu) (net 4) (status 1000000))
 (segment (start 53.397999 60.902001) (end 54.61 59.69) (width 0.5) (layer B.Cu) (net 4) (status 1000000))
 (segment (start 30.48 63.5) (end 30.48 59.351238) (width 0.25) (layer F.Cu) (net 5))
 (via (at 30.48 41.275) (size 0.8) (drill 0.4) (layers F.Cu B.Cu) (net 5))
 (segment (start 30.48 59.351238) (end 30.48 41.275) (width 0.25) (layer F.Cu) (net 5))
 (segment (start 32.837001 38.917999) (end 32.837001 31.567001) (width 0.25) (layer B.Cu) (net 5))
 (segment (start 32.837001 31.567001) (end 31.75 30.48) (width 0.25) (layer B.Cu) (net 5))
 (segment (start 30.48 41.275) (end 32.837001 38.917999) (width 0.25) (layer B.Cu) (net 5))
 (segment (start 30.537999 29.915999) (end 32.513998 27.94) (width 0.5) (layer F.Cu) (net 6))
 (segment (start 22.917999 42.375763) (end 30.537999 34.755763) (width 0.5) (layer F.Cu) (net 6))
 (segment (start 22.917999 64.598001) (end 22.917999 42.375763) (width 0.5) (layer F.Cu) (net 6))
 (segment (start 30.537999 34.755763) (end 30.537999 29.915999) (width 0.5) (layer F.Cu) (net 6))
 (segment (start 25.559999 67.240001) (end 22.917999 64.598001) (width 0.5) (layer F.Cu) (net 6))
 (segment (start 28.009999 67.240001) (end 25.559999 67.240001) (width 0.5) (layer F.Cu) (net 6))
 (segment (start 32.513998 27.94) (end 33.02 27.94) (width 0.5) (layer F.Cu) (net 6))
 (segment (start 29.21 66.04) (end 28.009999 67.240001) (width 0.5) (layer F.Cu) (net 6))
 (segment (start 52.07 59.69) (end 52.07 34.29) (width 0.5) (layer F.Cu) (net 6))
 (segment (start 33.02 27.94) (end 35.56 25.4) (width 0.5) (layer F.Cu) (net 6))
 (segment (start 43.03 25.4) (end 35.56 25.4) (width 0.5) (layer F.Cu) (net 6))
 (segment (start 30.48 67.31) (end 41.91 67.31) (width 0.5) (layer F.Cu) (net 6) (status 1000000))
 (segment (start 29.21 66.04) (end 30.48 67.31) (width 0.5) (layer F.Cu) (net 6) (status 1000000))
 (segment (start 41.91 67.31) (end 44.45 67.31) (width 0.5) (layer F.Cu) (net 6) (status 1000000))
 (segment (start 44.45 67.31) (end 52.07 59.69) (width 0.5) (layer F.Cu) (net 6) (status 1000000))
 (segment (start 35.377001 31.567001) (end 34.29 30.48) (width 0.25) (layer F.Cu) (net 7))
 (segment (start 35.377001 34.811761) (end 35.377001 31.567001) (width 0.25) (layer F.Cu) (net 7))
 (segment (start 27.94 42.248762) (end 35.377001 34.811761) (width 0.25) (layer F.Cu) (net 7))
 (segment (start 27.94 63.5) (end 27.94 42.248762) (width 0.25) (layer F.Cu) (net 7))
 (segment (start 27.94 66.361002) (end 30.158998 68.58) (width 0.25) (layer B.Cu) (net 7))
 (segment (start 27.94 63.5) (end 27.94 66.361002) (width 0.25) (layer B.Cu) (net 7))
 (segment (start 39.37 68.58) (end 41.91 71.12) (width 0.25) (layer B.Cu) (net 7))
 (segment (start 30.158998 68.58) (end 39.37 68.58) (width 0.25) (layer B.Cu) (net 7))
 (segment (start 34.56 27.94) (end 35.56 27.94) (width 0.25) (layer F.Cu) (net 8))
 (segment (start 33.202999 29.297001) (end 34.56 27.94) (width 0.25) (layer F.Cu) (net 8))
 (segment (start 33.202999 34.445763) (end 33.202999 29.297001) (width 0.25) (layer F.Cu) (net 8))
 (segment (start 25.582999 42.065763) (end 33.202999 34.445763) (width 0.25) (layer F.Cu) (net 8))
 (segment (start 25.582999 64.952999) (end 25.582999 42.065763) (width 0.25) (layer F.Cu) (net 8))
 (segment (start 26.67 66.04) (end 25.582999 64.952999) (width 0.25) (layer F.Cu) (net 8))
 (segment (start 55.245 31.115) (end 49.53 25.4) (width 0.25) (layer F.Cu) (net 9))
 (segment (start 62.23 31.115) (end 55.245 31.115) (width 0.25) (layer F.Cu) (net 9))
 (segment (start 52.07 31.75) (end 52.07 31.115) (width 0.25) (layer F.Cu) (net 22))
 (segment (start 49.53 34.29) (end 52.07 31.75) (width 0.25) (layer F.Cu) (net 22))
 (segment (start 52.07 71.12) (end 52.07 67.31) (width 0.25) (layer B.Cu) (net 19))
 (segment (start 52.07 67.31) (end 55.697001 63.682999) (width 0.25) (layer B.Cu) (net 19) (status 1000000))
 (segment (start 55.697001 63.682999) (end 55.697001 48.077001) (width 0.25) (layer B.Cu) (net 19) (status 1000000))
 (segment (start 55.697001 48.077001) (end 41.91 34.29) (width 0.25) (layer B.Cu) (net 19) (status 1000000)))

